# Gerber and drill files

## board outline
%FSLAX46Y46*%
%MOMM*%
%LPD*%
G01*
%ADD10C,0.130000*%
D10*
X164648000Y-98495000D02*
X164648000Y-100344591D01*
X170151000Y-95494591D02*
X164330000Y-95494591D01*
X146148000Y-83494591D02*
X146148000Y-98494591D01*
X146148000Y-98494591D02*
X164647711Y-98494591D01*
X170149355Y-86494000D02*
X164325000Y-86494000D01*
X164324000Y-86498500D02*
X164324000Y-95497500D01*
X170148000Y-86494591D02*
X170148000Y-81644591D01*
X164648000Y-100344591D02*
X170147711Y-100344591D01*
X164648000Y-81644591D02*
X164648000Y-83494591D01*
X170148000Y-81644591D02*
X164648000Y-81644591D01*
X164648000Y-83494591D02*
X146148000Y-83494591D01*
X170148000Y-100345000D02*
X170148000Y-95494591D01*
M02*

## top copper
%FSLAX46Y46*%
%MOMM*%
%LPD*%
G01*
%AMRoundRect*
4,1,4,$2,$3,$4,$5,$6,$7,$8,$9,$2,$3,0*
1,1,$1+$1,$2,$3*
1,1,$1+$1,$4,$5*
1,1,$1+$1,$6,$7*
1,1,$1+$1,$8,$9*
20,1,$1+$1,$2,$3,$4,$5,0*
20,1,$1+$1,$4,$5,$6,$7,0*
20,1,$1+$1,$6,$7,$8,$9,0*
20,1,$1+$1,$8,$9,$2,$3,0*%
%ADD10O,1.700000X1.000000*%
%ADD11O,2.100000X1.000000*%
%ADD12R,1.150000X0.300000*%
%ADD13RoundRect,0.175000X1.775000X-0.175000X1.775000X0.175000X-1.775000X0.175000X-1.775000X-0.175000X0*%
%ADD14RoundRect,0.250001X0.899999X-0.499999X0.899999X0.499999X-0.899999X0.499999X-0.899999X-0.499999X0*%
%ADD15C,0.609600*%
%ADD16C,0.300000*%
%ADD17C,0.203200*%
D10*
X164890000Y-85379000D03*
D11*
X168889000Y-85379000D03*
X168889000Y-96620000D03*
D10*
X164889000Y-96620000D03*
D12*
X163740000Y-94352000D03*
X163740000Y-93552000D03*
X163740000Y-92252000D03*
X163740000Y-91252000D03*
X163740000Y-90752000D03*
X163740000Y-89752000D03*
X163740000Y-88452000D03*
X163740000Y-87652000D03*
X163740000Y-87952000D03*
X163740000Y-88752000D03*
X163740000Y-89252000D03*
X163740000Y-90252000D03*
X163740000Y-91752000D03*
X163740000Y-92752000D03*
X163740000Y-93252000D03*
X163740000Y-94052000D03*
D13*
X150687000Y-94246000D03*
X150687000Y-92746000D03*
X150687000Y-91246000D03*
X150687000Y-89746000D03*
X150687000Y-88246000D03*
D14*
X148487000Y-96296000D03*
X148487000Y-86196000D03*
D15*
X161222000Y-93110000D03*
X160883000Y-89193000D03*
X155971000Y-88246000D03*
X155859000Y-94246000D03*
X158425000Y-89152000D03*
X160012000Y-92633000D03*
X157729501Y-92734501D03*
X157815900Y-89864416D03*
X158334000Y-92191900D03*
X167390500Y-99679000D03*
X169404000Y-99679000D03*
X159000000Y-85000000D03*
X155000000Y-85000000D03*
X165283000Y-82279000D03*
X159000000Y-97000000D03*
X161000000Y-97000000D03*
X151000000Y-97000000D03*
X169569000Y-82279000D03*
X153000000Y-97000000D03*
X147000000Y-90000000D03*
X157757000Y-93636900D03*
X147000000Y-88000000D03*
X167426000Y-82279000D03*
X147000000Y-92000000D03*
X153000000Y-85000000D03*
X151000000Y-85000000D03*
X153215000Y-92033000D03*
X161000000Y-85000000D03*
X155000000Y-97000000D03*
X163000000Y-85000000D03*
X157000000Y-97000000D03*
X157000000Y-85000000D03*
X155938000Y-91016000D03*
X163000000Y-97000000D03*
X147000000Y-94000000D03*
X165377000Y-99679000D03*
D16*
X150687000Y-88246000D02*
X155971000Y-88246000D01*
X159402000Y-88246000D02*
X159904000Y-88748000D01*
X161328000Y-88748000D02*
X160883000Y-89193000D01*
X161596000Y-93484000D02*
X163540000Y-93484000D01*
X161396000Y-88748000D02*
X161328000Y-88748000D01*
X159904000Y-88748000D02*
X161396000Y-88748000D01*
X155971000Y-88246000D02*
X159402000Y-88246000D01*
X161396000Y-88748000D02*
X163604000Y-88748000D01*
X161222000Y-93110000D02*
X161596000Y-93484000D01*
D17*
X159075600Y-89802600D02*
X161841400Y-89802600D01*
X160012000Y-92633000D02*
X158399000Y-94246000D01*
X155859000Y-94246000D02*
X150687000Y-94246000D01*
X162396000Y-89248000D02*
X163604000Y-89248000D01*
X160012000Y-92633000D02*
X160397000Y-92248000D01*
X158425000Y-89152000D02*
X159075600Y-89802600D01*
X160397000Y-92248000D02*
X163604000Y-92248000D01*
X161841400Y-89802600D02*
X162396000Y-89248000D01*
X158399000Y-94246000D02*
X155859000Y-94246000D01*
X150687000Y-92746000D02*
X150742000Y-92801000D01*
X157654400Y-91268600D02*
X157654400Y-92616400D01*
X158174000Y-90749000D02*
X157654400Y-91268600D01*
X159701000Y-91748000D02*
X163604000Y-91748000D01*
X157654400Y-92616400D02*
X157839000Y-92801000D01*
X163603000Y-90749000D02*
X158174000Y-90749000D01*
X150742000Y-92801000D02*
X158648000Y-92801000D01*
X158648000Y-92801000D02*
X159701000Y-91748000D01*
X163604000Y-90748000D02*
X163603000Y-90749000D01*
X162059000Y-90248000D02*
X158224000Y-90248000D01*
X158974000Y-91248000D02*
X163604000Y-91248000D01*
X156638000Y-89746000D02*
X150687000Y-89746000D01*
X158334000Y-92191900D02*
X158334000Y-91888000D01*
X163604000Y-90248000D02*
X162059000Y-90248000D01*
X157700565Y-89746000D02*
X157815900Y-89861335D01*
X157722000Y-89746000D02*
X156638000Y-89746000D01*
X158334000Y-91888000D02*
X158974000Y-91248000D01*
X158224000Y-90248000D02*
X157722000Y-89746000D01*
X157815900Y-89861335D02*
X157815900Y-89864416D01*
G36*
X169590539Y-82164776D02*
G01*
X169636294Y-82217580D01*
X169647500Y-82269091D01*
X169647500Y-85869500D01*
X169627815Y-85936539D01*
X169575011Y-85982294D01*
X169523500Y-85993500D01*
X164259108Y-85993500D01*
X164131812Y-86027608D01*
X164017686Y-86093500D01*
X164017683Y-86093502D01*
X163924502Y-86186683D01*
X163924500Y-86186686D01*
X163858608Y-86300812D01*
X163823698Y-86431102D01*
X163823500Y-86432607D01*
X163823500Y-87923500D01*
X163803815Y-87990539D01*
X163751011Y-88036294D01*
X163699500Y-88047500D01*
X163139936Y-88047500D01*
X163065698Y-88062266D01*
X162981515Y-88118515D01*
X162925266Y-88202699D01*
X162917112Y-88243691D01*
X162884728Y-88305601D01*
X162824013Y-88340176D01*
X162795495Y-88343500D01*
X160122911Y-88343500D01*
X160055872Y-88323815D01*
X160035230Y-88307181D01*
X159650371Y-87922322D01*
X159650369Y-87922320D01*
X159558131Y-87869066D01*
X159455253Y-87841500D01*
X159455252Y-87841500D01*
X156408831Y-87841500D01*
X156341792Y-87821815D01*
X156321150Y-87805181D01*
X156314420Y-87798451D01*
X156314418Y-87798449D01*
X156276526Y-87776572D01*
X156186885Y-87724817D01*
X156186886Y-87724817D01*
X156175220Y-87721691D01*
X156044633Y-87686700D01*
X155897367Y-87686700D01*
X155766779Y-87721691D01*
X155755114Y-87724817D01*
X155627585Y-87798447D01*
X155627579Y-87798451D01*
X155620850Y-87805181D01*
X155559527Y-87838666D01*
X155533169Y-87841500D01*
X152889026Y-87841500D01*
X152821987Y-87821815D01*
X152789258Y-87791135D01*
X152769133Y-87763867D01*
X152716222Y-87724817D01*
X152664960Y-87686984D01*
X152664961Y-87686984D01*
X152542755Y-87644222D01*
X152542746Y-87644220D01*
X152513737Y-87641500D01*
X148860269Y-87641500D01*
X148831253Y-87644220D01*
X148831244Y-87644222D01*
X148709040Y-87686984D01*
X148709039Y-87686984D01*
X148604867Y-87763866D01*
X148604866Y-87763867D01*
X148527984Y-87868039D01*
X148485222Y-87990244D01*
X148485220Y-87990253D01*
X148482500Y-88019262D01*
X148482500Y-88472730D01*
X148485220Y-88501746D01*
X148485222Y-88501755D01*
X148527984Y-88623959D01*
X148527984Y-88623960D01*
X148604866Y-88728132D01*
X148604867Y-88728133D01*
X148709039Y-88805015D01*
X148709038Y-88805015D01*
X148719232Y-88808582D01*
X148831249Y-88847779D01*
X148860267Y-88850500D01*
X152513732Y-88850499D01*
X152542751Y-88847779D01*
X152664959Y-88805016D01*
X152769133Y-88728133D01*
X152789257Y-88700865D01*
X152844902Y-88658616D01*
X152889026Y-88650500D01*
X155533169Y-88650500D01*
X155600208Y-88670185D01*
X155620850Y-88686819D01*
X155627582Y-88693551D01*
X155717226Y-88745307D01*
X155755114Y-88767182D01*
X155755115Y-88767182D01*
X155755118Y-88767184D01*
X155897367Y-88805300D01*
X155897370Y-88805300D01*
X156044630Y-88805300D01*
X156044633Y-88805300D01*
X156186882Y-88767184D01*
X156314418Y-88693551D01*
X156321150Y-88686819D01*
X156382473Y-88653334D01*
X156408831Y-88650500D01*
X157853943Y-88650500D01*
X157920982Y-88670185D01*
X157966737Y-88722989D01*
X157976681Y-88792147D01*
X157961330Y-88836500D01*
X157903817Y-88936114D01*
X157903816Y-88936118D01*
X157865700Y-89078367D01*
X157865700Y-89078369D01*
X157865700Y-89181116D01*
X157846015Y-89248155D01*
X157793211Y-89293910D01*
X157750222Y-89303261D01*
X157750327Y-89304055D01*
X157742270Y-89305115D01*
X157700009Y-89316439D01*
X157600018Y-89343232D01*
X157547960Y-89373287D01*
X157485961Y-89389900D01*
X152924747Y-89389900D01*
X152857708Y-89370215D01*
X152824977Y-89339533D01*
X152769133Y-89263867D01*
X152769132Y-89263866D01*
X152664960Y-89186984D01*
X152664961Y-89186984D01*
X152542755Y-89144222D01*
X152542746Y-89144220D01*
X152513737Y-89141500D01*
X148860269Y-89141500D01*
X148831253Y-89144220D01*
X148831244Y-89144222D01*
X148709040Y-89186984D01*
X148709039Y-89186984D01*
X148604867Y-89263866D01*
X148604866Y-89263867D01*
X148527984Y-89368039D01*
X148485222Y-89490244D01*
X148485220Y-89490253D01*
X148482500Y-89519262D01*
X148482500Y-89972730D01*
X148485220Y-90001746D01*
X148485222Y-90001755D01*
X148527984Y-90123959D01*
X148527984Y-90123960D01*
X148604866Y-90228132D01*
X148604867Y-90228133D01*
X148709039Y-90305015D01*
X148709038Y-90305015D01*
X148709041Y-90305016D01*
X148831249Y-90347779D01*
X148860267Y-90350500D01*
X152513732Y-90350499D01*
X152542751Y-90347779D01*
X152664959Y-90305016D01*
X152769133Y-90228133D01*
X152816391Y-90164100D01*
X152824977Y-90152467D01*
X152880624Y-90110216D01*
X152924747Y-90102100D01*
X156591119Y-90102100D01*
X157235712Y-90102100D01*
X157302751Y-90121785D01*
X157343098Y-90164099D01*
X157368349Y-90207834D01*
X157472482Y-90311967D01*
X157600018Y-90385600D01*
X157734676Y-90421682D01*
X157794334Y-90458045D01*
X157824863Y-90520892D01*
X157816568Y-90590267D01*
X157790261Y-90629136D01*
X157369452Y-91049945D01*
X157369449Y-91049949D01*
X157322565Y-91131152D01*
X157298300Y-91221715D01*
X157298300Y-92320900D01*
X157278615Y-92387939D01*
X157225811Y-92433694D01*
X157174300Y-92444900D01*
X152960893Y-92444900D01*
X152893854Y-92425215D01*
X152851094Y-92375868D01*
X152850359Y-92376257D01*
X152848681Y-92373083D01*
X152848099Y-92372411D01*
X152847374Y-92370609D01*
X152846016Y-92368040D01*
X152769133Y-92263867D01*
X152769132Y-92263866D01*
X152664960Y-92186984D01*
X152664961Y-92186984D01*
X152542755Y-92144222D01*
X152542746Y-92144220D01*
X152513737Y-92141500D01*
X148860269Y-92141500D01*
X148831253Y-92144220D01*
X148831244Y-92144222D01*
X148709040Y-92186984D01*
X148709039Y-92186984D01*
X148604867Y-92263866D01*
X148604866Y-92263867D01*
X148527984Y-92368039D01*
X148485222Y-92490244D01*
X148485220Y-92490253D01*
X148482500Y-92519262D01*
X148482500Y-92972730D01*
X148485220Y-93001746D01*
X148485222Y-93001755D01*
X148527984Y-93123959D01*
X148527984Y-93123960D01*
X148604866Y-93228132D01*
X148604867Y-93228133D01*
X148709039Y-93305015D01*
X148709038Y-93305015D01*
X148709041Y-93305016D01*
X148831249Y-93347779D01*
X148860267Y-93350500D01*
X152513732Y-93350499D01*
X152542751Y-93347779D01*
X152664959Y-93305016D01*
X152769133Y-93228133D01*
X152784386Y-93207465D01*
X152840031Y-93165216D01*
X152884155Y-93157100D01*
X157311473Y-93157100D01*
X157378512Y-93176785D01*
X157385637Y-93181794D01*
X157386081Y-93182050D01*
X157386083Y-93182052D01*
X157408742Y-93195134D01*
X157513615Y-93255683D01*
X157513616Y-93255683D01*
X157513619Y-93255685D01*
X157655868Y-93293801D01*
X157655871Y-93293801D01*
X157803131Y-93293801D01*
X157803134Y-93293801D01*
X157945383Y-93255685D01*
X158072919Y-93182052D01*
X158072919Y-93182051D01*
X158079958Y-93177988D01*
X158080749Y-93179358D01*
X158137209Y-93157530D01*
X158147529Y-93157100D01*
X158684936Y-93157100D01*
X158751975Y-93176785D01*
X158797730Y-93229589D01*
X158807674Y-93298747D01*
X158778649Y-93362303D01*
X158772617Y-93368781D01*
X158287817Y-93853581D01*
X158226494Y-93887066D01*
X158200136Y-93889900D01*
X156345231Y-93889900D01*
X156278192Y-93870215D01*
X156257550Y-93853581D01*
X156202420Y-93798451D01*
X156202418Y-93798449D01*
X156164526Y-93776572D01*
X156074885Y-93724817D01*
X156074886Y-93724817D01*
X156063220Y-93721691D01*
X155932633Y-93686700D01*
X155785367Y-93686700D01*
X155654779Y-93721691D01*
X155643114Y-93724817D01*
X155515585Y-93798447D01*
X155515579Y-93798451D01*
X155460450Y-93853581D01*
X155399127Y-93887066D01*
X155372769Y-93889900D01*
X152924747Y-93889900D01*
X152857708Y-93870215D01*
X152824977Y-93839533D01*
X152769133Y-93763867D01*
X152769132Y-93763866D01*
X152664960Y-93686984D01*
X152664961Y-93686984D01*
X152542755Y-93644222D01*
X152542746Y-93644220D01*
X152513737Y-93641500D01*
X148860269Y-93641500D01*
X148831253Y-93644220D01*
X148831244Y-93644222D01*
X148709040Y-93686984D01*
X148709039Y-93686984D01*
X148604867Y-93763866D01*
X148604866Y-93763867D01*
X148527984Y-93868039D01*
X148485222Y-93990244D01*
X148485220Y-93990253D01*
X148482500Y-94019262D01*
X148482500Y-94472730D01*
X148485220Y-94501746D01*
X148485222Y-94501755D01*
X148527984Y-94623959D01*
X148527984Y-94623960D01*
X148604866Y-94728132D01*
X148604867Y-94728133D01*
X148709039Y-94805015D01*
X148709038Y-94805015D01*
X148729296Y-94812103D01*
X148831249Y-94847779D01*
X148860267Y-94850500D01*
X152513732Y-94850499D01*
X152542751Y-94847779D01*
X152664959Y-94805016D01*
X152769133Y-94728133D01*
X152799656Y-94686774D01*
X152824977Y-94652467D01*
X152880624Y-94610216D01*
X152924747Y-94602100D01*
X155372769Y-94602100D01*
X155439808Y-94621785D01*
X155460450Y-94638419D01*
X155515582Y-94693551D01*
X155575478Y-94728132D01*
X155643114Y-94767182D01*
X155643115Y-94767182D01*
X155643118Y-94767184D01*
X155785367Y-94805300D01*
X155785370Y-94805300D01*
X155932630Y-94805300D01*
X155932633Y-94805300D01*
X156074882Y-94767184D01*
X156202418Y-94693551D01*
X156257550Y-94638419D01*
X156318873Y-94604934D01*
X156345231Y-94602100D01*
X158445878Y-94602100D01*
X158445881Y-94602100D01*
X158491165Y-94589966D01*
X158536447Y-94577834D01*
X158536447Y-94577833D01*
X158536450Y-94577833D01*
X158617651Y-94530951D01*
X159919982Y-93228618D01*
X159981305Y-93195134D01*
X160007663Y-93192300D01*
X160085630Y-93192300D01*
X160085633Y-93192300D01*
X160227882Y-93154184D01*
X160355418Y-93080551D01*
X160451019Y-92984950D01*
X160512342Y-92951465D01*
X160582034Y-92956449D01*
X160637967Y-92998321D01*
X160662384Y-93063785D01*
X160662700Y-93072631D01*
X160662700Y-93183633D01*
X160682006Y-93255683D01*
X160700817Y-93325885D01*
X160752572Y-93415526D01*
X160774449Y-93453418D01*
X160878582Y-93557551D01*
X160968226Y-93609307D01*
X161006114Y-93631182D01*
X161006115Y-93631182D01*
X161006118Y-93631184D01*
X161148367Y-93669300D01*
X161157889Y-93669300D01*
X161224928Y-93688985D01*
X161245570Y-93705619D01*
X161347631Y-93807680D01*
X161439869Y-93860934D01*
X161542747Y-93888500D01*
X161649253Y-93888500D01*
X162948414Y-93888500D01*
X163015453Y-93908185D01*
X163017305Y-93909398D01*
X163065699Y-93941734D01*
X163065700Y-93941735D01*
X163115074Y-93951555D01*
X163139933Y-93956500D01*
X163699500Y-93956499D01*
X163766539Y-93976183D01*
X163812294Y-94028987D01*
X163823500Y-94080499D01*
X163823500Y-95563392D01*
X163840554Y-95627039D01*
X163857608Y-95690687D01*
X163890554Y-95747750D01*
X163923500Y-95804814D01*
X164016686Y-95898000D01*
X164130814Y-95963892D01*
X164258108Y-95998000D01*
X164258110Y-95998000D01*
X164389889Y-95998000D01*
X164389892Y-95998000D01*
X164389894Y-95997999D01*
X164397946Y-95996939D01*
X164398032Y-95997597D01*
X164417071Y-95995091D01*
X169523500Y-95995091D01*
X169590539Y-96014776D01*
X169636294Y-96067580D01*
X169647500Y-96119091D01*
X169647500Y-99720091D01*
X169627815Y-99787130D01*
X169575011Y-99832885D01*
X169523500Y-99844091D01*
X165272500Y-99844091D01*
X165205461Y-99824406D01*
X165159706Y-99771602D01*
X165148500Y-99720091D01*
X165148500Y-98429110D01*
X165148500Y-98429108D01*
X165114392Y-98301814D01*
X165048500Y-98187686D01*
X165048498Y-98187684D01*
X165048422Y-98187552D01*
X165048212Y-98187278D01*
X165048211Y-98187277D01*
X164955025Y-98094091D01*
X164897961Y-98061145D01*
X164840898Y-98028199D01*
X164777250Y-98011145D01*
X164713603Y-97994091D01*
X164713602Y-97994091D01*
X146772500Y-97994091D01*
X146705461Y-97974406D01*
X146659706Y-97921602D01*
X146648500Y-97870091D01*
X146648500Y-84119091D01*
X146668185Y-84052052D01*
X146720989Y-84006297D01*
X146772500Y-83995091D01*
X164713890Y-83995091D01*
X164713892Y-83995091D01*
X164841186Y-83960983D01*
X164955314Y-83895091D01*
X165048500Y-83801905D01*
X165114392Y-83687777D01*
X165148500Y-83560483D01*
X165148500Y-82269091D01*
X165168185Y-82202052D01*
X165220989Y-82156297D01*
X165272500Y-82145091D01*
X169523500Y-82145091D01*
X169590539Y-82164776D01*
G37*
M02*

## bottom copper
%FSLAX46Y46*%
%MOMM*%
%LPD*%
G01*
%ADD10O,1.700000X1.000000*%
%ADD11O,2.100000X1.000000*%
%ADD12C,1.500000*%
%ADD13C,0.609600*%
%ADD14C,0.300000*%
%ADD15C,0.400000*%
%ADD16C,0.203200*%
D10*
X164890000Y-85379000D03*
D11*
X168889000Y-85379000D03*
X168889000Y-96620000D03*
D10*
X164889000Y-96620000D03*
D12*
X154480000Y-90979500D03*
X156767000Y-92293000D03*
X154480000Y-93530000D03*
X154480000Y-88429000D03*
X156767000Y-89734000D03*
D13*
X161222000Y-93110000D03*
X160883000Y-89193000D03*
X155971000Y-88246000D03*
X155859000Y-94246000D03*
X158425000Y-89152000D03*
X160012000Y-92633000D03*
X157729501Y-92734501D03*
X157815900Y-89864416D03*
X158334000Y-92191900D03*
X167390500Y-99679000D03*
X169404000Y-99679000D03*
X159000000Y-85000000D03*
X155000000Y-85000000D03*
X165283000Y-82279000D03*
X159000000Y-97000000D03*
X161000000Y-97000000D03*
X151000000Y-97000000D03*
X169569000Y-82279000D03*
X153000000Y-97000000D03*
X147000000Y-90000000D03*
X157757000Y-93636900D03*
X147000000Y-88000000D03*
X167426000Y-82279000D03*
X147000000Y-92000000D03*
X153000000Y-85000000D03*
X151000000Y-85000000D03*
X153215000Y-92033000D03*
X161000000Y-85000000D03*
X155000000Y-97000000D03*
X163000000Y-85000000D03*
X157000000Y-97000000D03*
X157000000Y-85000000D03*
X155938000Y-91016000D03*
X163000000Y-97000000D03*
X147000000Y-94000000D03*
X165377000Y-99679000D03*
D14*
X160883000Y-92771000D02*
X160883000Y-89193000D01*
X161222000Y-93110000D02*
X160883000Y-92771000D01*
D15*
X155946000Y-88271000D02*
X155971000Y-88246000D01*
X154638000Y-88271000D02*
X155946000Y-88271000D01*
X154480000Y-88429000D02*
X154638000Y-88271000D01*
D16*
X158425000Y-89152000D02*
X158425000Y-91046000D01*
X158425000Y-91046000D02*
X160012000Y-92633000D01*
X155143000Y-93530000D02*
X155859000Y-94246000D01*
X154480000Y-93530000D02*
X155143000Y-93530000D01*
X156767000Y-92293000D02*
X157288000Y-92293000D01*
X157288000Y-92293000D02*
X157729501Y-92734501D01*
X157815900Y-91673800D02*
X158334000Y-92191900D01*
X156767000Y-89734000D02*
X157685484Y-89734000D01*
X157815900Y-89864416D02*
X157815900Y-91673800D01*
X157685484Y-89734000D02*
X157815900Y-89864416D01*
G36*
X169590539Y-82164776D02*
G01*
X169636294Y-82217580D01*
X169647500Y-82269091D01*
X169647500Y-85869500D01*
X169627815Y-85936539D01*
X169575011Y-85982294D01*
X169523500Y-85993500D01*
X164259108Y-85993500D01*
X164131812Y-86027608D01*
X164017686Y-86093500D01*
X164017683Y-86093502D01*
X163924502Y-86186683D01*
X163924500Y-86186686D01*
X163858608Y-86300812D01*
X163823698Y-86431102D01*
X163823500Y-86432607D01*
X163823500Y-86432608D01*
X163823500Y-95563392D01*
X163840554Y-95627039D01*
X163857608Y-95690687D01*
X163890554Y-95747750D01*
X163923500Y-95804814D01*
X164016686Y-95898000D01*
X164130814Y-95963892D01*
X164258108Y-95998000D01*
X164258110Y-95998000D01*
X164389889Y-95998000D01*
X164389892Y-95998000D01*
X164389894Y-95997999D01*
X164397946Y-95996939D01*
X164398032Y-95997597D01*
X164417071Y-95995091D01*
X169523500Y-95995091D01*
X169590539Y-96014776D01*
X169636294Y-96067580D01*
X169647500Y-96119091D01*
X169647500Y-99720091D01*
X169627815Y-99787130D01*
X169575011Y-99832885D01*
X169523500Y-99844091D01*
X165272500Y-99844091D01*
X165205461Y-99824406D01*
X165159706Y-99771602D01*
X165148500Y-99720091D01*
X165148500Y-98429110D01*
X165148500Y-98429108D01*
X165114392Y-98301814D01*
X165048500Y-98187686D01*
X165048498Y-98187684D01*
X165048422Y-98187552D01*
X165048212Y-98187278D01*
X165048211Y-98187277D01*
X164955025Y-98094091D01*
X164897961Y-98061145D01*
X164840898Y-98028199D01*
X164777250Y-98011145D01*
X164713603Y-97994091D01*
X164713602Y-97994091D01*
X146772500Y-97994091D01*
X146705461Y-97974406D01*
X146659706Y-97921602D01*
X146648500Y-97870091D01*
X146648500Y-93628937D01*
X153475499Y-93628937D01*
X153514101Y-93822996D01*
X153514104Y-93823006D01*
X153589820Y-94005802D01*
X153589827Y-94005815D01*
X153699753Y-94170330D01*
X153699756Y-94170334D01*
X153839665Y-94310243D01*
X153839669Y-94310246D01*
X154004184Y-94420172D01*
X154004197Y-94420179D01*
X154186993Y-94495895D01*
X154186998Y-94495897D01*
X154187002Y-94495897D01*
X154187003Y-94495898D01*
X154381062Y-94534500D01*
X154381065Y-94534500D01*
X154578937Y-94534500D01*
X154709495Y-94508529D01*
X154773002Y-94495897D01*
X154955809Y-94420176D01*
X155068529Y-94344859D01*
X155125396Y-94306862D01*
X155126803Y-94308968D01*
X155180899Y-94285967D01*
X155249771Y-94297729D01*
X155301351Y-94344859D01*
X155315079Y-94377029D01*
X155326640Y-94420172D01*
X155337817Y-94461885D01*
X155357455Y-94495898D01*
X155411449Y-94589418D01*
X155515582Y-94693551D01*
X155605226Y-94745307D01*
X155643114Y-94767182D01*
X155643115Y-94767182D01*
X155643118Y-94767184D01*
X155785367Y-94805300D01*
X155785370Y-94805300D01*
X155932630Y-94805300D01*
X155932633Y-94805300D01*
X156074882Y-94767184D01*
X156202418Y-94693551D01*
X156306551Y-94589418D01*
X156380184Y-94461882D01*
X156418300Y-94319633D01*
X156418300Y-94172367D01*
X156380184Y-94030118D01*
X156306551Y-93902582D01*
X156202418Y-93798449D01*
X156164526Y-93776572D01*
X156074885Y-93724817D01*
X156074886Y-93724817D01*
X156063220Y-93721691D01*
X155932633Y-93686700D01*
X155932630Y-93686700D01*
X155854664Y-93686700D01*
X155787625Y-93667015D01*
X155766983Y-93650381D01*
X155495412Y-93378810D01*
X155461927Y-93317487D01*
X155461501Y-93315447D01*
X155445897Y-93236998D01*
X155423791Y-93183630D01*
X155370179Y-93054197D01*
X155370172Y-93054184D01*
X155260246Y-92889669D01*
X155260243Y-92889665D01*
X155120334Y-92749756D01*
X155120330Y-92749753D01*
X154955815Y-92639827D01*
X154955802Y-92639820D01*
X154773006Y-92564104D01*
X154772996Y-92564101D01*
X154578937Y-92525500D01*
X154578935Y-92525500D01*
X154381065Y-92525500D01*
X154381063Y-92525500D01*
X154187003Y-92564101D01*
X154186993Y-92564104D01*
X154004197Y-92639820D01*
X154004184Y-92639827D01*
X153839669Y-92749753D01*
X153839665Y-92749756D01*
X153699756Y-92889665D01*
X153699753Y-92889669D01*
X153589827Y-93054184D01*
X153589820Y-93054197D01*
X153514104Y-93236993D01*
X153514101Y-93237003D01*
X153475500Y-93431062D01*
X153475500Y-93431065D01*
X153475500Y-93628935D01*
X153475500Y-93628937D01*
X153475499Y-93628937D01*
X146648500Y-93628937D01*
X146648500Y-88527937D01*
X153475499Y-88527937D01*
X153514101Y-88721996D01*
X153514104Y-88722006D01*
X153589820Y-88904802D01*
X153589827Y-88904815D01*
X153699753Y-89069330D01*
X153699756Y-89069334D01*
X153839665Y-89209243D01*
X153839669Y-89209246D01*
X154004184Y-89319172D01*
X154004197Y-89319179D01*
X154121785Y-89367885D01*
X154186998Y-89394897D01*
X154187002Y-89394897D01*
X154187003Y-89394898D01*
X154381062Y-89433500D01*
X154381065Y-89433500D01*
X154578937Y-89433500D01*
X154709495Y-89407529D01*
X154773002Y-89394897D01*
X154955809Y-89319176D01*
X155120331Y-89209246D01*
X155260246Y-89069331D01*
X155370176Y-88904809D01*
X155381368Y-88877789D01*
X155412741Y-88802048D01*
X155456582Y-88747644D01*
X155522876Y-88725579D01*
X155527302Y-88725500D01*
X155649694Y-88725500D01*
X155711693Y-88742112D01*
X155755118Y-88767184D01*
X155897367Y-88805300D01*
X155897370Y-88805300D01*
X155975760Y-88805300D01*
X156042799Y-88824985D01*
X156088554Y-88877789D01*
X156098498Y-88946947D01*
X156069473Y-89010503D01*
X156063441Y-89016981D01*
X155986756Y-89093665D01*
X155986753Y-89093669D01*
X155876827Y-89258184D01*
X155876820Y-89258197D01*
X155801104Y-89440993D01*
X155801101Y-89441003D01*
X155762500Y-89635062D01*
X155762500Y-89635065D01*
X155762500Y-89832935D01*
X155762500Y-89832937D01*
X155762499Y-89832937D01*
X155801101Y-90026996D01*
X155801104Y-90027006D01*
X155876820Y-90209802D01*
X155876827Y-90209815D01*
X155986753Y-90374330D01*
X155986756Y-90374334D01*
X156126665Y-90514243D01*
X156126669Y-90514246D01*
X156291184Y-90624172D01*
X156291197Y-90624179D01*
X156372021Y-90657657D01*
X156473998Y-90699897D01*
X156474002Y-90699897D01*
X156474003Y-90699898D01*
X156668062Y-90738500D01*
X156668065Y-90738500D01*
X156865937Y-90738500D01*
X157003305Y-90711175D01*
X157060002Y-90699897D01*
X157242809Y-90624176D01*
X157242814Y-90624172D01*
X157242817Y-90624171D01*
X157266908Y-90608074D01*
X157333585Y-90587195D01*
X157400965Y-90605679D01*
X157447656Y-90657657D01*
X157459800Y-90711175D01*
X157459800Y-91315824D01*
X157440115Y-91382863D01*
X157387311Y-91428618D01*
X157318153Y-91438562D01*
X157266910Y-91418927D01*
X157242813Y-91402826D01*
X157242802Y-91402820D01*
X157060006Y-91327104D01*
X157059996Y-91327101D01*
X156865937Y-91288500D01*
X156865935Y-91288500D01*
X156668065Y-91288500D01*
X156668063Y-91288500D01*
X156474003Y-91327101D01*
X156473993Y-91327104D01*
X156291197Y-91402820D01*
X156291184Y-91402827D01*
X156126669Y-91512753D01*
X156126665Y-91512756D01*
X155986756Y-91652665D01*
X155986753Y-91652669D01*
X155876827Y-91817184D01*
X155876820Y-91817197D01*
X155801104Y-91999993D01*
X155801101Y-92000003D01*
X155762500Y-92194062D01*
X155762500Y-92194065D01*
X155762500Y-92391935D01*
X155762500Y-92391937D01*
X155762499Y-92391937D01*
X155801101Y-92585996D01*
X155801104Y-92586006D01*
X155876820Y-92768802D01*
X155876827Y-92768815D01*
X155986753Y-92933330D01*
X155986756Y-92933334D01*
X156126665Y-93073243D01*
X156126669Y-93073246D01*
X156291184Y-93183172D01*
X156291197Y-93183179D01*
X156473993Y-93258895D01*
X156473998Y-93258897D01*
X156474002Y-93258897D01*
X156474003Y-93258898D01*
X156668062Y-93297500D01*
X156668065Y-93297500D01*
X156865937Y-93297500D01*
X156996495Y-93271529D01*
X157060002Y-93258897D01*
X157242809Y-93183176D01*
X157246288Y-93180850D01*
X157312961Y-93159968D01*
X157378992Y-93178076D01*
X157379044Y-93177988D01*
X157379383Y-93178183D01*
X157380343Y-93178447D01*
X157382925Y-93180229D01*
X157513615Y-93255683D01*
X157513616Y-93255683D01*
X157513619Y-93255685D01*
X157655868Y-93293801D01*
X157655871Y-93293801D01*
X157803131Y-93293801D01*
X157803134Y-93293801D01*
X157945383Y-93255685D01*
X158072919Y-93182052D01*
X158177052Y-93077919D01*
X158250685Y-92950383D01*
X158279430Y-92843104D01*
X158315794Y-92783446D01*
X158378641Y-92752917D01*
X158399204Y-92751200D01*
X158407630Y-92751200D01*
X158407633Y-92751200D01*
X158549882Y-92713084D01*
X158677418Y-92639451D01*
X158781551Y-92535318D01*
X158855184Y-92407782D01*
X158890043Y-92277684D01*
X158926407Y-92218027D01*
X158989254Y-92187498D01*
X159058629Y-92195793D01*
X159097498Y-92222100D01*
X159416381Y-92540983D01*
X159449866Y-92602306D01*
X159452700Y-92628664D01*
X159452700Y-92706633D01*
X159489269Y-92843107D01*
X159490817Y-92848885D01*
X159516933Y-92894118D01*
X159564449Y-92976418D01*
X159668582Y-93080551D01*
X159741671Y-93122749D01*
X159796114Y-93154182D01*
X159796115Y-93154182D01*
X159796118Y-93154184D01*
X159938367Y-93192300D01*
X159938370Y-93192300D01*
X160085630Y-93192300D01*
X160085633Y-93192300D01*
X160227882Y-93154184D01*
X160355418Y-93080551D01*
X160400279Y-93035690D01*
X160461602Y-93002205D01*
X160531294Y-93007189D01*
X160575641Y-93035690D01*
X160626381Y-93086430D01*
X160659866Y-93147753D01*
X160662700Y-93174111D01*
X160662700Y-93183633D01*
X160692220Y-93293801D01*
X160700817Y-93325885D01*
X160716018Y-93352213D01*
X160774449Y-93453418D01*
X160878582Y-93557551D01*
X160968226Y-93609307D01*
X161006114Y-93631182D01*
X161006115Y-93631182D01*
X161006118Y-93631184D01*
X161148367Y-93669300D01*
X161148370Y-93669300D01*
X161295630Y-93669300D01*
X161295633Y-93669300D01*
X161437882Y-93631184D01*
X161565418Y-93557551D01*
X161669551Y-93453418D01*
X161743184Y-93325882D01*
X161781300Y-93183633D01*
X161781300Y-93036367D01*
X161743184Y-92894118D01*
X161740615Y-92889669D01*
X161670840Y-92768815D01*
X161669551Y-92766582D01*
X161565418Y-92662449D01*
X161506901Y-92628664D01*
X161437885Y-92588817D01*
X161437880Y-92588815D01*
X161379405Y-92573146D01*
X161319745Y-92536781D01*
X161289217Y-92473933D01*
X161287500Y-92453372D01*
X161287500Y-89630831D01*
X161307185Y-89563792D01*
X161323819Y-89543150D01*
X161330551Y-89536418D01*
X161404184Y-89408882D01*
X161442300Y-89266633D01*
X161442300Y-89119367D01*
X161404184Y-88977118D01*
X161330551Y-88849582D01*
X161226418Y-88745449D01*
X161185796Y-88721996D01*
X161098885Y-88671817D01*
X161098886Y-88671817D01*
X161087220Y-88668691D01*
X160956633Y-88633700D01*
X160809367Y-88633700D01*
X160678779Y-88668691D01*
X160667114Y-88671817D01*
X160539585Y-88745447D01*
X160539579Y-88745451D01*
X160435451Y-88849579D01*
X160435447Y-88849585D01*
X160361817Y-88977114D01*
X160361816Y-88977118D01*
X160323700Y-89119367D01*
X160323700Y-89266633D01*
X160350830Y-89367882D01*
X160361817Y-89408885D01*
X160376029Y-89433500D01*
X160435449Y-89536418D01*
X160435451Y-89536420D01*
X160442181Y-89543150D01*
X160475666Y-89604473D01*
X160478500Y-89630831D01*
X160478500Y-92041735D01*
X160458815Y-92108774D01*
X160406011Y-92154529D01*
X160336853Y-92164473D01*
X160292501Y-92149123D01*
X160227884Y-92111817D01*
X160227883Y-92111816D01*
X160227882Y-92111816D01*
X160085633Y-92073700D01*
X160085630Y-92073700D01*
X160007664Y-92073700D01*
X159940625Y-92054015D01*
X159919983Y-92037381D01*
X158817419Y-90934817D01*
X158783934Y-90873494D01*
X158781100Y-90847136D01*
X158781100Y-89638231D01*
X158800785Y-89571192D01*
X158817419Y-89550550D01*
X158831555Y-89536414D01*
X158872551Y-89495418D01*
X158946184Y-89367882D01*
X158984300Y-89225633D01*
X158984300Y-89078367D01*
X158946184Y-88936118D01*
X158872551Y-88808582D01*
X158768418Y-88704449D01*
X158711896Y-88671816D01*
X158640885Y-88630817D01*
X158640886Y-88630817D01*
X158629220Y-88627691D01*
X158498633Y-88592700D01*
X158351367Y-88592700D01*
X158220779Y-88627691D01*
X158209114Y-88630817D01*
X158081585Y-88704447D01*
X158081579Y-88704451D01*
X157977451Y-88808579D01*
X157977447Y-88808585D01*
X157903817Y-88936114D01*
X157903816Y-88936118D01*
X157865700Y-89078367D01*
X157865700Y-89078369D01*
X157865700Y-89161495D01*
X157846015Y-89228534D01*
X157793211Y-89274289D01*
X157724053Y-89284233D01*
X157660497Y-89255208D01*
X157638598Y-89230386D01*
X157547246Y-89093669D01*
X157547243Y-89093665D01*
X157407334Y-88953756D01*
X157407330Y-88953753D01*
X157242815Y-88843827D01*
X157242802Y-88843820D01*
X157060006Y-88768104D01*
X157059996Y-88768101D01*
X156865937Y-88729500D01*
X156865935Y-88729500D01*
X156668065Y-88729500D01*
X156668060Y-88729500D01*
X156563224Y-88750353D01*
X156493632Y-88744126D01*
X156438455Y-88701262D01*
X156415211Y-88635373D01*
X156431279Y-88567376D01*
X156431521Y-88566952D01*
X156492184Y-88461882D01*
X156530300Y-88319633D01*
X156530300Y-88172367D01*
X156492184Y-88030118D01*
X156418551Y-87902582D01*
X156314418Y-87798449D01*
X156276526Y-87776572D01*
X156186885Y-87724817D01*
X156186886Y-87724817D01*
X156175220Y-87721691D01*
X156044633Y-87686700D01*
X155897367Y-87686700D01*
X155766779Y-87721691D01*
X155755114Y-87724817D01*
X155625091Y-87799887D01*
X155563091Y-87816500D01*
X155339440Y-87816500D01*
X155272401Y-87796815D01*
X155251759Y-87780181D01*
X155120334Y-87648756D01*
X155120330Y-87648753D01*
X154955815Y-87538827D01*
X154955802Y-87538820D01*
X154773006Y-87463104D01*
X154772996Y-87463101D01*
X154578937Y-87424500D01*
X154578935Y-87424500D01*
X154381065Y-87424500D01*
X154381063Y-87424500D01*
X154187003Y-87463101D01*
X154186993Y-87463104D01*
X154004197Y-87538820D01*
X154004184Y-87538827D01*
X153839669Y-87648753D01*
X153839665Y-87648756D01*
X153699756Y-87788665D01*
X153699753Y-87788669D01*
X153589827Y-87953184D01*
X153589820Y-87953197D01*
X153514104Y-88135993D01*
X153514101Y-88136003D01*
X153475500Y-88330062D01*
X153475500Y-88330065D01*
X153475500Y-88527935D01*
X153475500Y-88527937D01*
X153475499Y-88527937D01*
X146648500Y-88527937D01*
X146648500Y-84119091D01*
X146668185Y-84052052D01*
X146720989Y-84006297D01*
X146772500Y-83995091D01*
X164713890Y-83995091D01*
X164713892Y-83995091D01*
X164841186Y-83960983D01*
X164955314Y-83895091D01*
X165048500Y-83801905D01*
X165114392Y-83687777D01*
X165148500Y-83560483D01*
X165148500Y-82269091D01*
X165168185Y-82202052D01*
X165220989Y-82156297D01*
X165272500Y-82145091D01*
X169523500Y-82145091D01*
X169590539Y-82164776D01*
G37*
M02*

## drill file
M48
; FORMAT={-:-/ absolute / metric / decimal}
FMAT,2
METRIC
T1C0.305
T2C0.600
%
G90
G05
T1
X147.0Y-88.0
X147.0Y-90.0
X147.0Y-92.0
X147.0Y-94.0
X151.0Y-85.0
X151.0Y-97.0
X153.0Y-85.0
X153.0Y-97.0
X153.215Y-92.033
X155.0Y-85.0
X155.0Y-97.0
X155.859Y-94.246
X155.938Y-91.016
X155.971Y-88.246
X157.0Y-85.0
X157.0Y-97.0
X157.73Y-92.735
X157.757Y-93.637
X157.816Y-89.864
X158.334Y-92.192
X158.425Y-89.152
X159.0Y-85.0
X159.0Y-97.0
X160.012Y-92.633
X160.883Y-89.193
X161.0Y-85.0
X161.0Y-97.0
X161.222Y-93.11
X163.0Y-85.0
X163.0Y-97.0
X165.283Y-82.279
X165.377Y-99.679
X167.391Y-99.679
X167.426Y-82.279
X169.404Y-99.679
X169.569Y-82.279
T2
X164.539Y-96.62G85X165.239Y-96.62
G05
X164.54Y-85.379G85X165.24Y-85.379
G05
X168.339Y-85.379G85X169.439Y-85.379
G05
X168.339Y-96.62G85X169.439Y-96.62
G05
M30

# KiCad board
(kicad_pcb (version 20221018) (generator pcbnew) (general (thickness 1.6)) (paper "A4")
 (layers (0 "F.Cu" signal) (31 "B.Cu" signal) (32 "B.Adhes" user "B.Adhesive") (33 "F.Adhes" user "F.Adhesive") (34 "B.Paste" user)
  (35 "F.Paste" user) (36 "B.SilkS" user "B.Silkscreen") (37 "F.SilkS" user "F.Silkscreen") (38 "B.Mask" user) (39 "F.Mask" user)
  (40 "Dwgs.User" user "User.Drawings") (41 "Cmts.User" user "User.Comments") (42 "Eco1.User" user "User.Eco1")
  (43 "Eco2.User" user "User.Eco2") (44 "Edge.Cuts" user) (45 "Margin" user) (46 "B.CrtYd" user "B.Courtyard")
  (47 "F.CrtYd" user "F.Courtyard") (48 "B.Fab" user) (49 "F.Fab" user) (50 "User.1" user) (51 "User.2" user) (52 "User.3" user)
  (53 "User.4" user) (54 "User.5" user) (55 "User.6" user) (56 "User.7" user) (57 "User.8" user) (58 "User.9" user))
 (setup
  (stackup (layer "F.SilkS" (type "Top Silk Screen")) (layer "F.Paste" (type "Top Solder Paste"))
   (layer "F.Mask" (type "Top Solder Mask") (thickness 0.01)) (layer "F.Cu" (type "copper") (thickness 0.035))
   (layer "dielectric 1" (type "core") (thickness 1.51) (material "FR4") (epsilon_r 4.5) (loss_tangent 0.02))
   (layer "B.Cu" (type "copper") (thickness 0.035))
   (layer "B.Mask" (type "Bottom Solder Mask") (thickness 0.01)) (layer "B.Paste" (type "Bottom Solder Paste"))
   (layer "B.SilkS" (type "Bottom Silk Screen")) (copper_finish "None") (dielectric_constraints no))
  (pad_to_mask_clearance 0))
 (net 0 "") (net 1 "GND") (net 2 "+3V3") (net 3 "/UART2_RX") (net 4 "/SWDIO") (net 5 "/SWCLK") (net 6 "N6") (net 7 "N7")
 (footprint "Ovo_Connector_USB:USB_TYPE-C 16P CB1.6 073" (layer "F.Cu") (at 167.41 91.002 90)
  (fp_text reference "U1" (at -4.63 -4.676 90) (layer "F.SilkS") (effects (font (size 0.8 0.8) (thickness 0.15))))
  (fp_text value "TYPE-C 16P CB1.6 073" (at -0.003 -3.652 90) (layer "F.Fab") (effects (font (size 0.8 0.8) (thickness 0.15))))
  (pad "25" thru_hole oval (at 5.623 -2.52 90) (size 1 1.7) (drill oval 0.6 1.3) (layers "*.Cu" "*.Mask") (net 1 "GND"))
  (pad "26" thru_hole oval (at 5.623 1.479 90) (size 1 2.1) (drill oval 0.6 1.7) (layers "*.Cu" "*.Mask") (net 1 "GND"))
  (pad "27" thru_hole oval (at -5.618 1.479 90) (size 1 2.1) (drill oval 0.6 1.7) (layers "*.Cu" "*.Mask") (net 1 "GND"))
  (pad "28" thru_hole oval (at -5.618 -2.521 90) (size 1 1.7) (drill oval 0.6 1.3) (layers "*.Cu" "*.Mask") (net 1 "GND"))
  (pad "A1" smd rect (at -3.35 -3.67 90) (size 0.3 1.15) (layers "F.Cu" "F.Paste" "F.Mask") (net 1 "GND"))
  (pad "A4" smd rect (at -2.55 -3.67 90) (size 0.3 1.15) (layers "F.Cu" "F.Paste" "F.Mask") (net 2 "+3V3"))
  (pad "A5" smd rect (at -1.25 -3.67 90) (size 0.3 1.15) (layers "F.Cu" "F.Paste" "F.Mask") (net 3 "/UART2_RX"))
  (pad "A6" smd rect (at -0.25 -3.67 90) (size 0.3 1.15) (layers "F.Cu" "F.Paste" "F.Mask") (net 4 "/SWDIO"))
  (pad "A7" smd rect (at 0.25 -3.67 90) (size 0.3 1.15) (layers "F.Cu" "F.Paste" "F.Mask") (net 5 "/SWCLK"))
  (pad "A8" smd rect (at 1.25 -3.67 90) (size 0.3 1.15) (layers "F.Cu" "F.Paste" "F.Mask") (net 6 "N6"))
  (pad "A9" smd rect (at 2.55 -3.67 90) (size 0.3 1.15) (layers "F.Cu" "F.Paste" "F.Mask") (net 2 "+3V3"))
  (pad "A12" smd rect (at 3.35 -3.67 90) (size 0.3 1.15) (layers "F.Cu" "F.Paste" "F.Mask") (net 1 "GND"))
  (pad "B1" smd rect (at 3.05 -3.67 90) (size 0.3 1.15) (layers "F.Cu" "F.Paste" "F.Mask") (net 1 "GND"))
  (pad "B4" smd rect (at 2.25 -3.67 90) (size 0.3 1.15) (layers "F.Cu" "F.Paste" "F.Mask") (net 2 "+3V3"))
  (pad "B5" smd rect (at 1.75 -3.67 90) (size 0.3 1.15) (layers "F.Cu" "F.Paste" "F.Mask") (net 3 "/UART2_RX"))
  (pad "B6" smd rect (at 0.75 -3.67 90) (size 0.3 1.15) (layers "F.Cu" "F.Paste" "F.Mask") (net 4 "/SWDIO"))
  (pad "B7" smd rect (at -0.75 -3.67 90) (size 0.3 1.15) (layers "F.Cu" "F.Paste" "F.Mask") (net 5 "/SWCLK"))
  (pad "B8" smd rect (at -1.75 -3.67 90) (size 0.3 1.15) (layers "F.Cu" "F.Paste" "F.Mask") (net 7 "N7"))
  (pad "B9" smd rect (at -2.25 -3.67 90) (size 0.3 1.15) (layers "F.Cu" "F.Paste" "F.Mask") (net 2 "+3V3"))
  (pad "B12" smd rect (at -3.05 -3.67 90) (size 0.3 1.15) (layers "F.Cu" "F.Paste" "F.Mask") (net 1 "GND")))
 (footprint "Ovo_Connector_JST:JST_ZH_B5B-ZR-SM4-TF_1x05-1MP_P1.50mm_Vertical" (layer "F.Cu") (at 149.987 91.246 90)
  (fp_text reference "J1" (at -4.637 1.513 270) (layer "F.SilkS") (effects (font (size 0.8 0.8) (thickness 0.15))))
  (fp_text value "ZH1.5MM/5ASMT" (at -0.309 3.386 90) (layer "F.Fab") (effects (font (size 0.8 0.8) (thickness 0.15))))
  (pad "1" smd roundrect (at -3 0.7 90) (size 0.7 3.9) (layers "F.Cu" "F.Paste" "F.Mask") (roundrect_rratio 0.25) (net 3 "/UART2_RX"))
  (pad "2" smd roundrect (at -1.5 0.7 90) (size 0.7 3.9) (layers "F.Cu" "F.Paste" "F.Mask") (roundrect_rratio 0.25) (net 5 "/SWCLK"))
  (pad "3" smd roundrect (at 0 0.7 90) (size 0.7 3.9) (layers "F.Cu" "F.Paste" "F.Mask") (roundrect_rratio 0.25) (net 1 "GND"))
  (pad "4" smd roundrect (at 1.5 0.7 90) (size 0.7 3.9) (layers "F.Cu" "F.Paste" "F.Mask") (roundrect_rratio 0.25) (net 4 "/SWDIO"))
  (pad "5" smd roundrect (at 3 0.7 90) (size 0.7 3.9) (layers "F.Cu" "F.Paste" "F.Mask") (roundrect_rratio 0.25) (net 2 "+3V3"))
  (pad "MP" smd roundrect (at -5.05 -1.5 90) (size 1.5 2.3) (layers "F.Cu" "F.Paste" "F.Mask") (roundrect_rratio 0.1666673333) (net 1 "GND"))
  (pad "MP" smd roundrect (at 5.05 -1.5 90) (size 1.5 2.3) (layers "F.Cu" "F.Paste" "F.Mask") (roundrect_rratio 0.1666673333) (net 1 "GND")))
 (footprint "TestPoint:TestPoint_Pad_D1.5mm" (layer "B.Cu") (at 154.48 90.9795 180)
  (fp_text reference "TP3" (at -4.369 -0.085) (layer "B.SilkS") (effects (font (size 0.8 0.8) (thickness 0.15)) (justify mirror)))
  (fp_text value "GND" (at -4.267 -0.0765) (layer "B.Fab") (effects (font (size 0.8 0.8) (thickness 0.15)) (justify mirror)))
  (pad "1" smd circle (at 0 0 180) (size 1.5 1.5) (layers "B.Cu" "B.Mask") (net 1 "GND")))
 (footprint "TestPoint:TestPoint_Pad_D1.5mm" (layer "B.Cu") (at 156.767 92.293 180)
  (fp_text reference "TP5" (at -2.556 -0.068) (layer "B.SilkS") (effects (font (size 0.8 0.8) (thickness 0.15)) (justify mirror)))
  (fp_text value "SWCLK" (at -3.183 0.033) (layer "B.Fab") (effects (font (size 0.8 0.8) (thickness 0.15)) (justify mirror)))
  (pad "1" smd circle (at 0 0 180) (size 1.5 1.5) (layers "B.Cu" "B.Mask") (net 5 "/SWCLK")))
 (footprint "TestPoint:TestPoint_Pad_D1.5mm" (layer "B.Cu") (at 154.48 93.53 180)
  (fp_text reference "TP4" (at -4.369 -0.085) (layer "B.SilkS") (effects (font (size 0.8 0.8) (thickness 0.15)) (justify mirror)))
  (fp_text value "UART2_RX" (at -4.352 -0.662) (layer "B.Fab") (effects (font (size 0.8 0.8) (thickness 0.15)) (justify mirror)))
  (pad "1" smd circle (at 0 0 180) (size 1.5 1.5) (layers "B.Cu" "B.Mask") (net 3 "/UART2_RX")))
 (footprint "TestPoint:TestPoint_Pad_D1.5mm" (layer "B.Cu") (at 154.48 88.429 180)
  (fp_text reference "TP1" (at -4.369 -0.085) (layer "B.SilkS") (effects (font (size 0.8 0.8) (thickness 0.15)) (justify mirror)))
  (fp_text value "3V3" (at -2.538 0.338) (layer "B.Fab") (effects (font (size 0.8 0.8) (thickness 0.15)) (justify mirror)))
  (pad "1" smd circle (at 0 0 180) (size 1.5 1.5) (layers "B.Cu" "B.Mask") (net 2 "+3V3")))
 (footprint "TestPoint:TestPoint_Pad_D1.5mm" (layer "B.Cu") (at 156.767 89.734 180)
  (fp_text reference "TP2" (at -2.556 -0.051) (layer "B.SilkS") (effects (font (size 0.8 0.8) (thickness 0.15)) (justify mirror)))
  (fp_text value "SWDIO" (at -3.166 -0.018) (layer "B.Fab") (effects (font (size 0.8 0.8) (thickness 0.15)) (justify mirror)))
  (pad "1" smd circle (at 0 0 180) (size 1.5 1.5) (layers "B.Cu" "B.Mask") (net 4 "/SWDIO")))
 (gr_line (start 164.648 98.495) (end 164.648 100.344591) (stroke (width 0.13) (type solid)) (layer "Edge.Cuts"))
 (gr_line (start 170.151 95.494591) (end 164.33 95.494591) (stroke (width 0.13) (type solid)) (layer "Edge.Cuts"))
 (gr_line (start 146.148 83.494591) (end 146.148 98.494591) (stroke (width 0.13) (type solid)) (layer "Edge.Cuts"))
 (gr_line (start 146.148 98.494591) (end 164.647711 98.494591) (stroke (width 0.13) (type solid)) (layer "Edge.Cuts"))
 (gr_line (start 170.149355 86.494) (end 164.325 86.494) (stroke (width 0.13) (type solid)) (layer "Edge.Cuts"))
 (gr_line (start 164.324 86.4985) (end 164.324 95.4975) (stroke (width 0.13) (type solid)) (layer "Edge.Cuts"))
 (gr_line (start 170.148 86.494591) (end 170.148 81.644591) (stroke (width 0.13) (type solid)) (layer "Edge.Cuts"))
 (gr_line (start 164.648 100.344591) (end 170.147711 100.344591) (stroke (width 0.13) (type solid)) (layer "Edge.Cuts"))
 (gr_line (start 164.648 81.644591) (end 164.648 83.494591) (stroke (width 0.13) (type solid)) (layer "Edge.Cuts"))
 (gr_line (start 170.148 81.644591) (end 164.648 81.644591) (stroke (width 0.13) (type solid)) (layer "Edge.Cuts"))
 (gr_line (start 164.648 83.494591) (end 146.148 83.494591) (stroke (width 0.13) (type solid)) (layer "Edge.Cuts"))
 (gr_line (start 170.148 100.345) (end 170.148 95.494591) (stroke (width 0.13) (type solid)) (layer "Edge.Cuts"))
 (segment (start 150.687 88.246) (end 155.971 88.246) (width 0.3) (layer "F.Cu") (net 2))
 (segment (start 159.402 88.246) (end 159.904 88.748) (width 0.3) (layer "F.Cu") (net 2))
 (segment (start 161.328 88.748) (end 160.883 89.193) (width 0.3) (layer "F.Cu") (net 2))
 (segment (start 161.596 93.484) (end 163.54 93.484) (width 0.3) (layer "F.Cu") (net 2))
 (segment (start 161.396 88.748) (end 161.328 88.748) (width 0.3) (layer "F.Cu") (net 2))
 (segment (start 159.904 88.748) (end 161.396 88.748) (width 0.3) (layer "F.Cu") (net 2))
 (segment (start 155.971 88.246) (end 159.402 88.246) (width 0.3) (layer "F.Cu") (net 2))
 (segment (start 161.396 88.748) (end 163.604 88.748) (width 0.3) (layer "F.Cu") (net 2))
 (segment (start 161.222 93.11) (end 161.596 93.484) (width 0.3) (layer "F.Cu") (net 2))
 (via (at 161.222 93.11) (size 0.6096) (drill 0.3048) (layers "F.Cu" "B.Cu") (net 2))
 (via (at 160.883 89.193) (size 0.6096) (drill 0.3048) (layers "F.Cu" "B.Cu") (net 2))
 (via (at 155.971 88.246) (size 0.6096) (drill 0.3048) (layers "F.Cu" "B.Cu") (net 2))
 (segment (start 160.883 92.771) (end 160.883 89.193) (width 0.3) (layer "B.Cu") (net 2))
 (segment (start 161.222 93.11) (end 160.883 92.771) (width 0.3) (layer "B.Cu") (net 2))
 (segment (start 155.946 88.271) (end 155.971 88.246) (width 0.4) (layer "B.Cu") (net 2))
 (segment (start 154.638 88.271) (end 155.946 88.271) (width 0.4) (layer "B.Cu") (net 2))
 (segment (start 154.48 88.429) (end 154.638 88.271) (width 0.4) (layer "B.Cu") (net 2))
 (segment (start 159.0756 89.8026) (end 161.8414 89.8026) (width 0.2032) (layer "F.Cu") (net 3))
 (segment (start 160.012 92.633) (end 158.399 94.246) (width 0.2032) (layer "F.Cu") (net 3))
 (segment (start 155.859 94.246) (end 150.687 94.246) (width 0.2032) (layer "F.Cu") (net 3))
 (segment (start 162.396 89.248) (end 163.604 89.248) (width 0.2032) (layer "F.Cu") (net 3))
 (segment (start 160.012 92.633) (end 160.397 92.248) (width 0.2032) (layer "F.Cu") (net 3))
 (segment (start 158.425 89.152) (end 159.0756 89.8026) (width 0.2032) (layer "F.Cu") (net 3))
 (segment (start 160.397 92.248) (end 163.604 92.248) (width 0.2032) (layer "F.Cu") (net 3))
 (segment (start 161.8414 89.8026) (end 162.396 89.248) (width 0.2032) (layer "F.Cu") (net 3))
 (segment (start 158.399 94.246) (end 155.859 94.246) (width 0.2032) (layer "F.Cu") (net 3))
 (via (at 155.859 94.246) (size 0.6096) (drill 0.3048) (layers "F.Cu" "B.Cu") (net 3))
 (via (at 158.425 89.152) (size 0.6096) (drill 0.3048) (layers "F.Cu" "B.Cu") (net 3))
 (via (at 160.012 92.633) (size 0.6096) (drill 0.3048) (layers "F.Cu" "B.Cu") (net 3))
 (segment (start 158.425 89.152) (end 158.425 91.046) (width 0.2032) (layer "B.Cu") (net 3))
 (segment (start 158.425 91.046) (end 160.012 92.633) (width 0.2032) (layer "B.Cu") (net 3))
 (segment (start 155.143 93.53) (end 155.859 94.246) (width 0.2032) (layer "B.Cu") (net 3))
 (segment (start 154.48 93.53) (end 155.143 93.53) (width 0.2032) (layer "B.Cu") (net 3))
 (segment (start 150.687 92.746) (end 150.742 92.801) (width 0.2032) (layer "F.Cu") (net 5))
 (segment (start 157.6544 91.2686) (end 157.6544 92.6164) (width 0.2032) (layer "F.Cu") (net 5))
 (segment (start 158.174 90.749) (end 157.6544 91.2686) (width 0.2032) (layer "F.Cu") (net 5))
 (segment (start 159.701 91.748) (end 163.604 91.748) (width 0.2032) (layer "F.Cu") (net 5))
 (segment (start 157.6544 92.6164) (end 157.839 92.801) (width 0.2032) (layer "F.Cu") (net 5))
 (segment (start 163.603 90.749) (end 158.174 90.749) (width 0.2032) (layer "F.Cu") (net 5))
 (segment (start 150.742 92.801) (end 158.648 92.801) (width 0.2032) (layer "F.Cu") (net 5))
 (segment (start 158.648 92.801) (end 159.701 91.748) (width 0.2032) (layer "F.Cu") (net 5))
 (segment (start 163.604 90.748) (end 163.603 90.749) (width 0.2032) (layer "F.Cu") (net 5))
 (via (at 157.729501 92.734501) (size 0.6096) (drill 0.3048) (layers "F.Cu" "B.Cu") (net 5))
 (segment (start 156.767 92.293) (end 157.288 92.293) (width 0.2032) (layer "B.Cu") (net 5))
 (segment (start 157.288 92.293) (end 157.729501 92.734501) (width 0.2032) (layer "B.Cu") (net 5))
 (segment (start 162.059 90.248) (end 158.224 90.248) (width 0.2032) (layer "F.Cu") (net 4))
 (segment (start 158.974 91.248) (end 163.604 91.248) (width 0.2032) (layer "F.Cu") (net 4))
 (segment (start 156.638 89.746) (end 150.687 89.746) (width 0.2032) (layer "F.Cu") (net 4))
 (segment (start 158.334 92.1919) (end 158.334 91.888) (width 0.2032) (layer "F.Cu") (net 4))
 (segment (start 163.604 90.248) (end 162.059 90.248) (width 0.2032) (layer "F.Cu") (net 4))
 (segment (start 157.700565 89.746) (end 157.8159 89.861335) (width 0.2032) (layer "F.Cu") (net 4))
 (segment (start 157.722 89.746) (end 156.638 89.746) (width 0.2032) (layer "F.Cu") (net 4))
 (segment (start 158.334 91.888) (end 158.974 91.248) (width 0.2032) (layer "F.Cu") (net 4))
 (segment (start 158.224 90.248) (end 157.722 89.746) (width 0.2032) (layer "F.Cu") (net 4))
 (segment (start 157.8159 89.861335) (end 157.8159 89.864416) (width 0.2032) (layer "F.Cu") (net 4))
 (via (at 157.8159 89.864416) (size 0.6096) (drill 0.3048) (layers "F.Cu" "B.Cu") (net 4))
 (via (at 158.334 92.1919) (size 0.6096) (drill 0.3048) (layers "F.Cu" "B.Cu") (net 4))
 (segment (start 157.8159 91.6738) (end 158.334 92.1919) (width 0.2032) (layer "B.Cu") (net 4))
 (segment (start 156.767 89.734) (end 157.685484 89.734) (width 0.2032) (layer "B.Cu") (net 4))
 (segment (start 157.8159 89.864416) (end 157.8159 91.6738) (width 0.2032) (layer "B.Cu") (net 4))
 (segment (start 157.685484 89.734) (end 157.8159 89.864416) (width 0.2032) (layer "B.Cu") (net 4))
 (via (at 167.3905 99.679) (size 0.6096) (drill 0.3048) (layers "F.Cu" "B.Cu") (free) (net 1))
 (via (at 169.404 99.679) (size 0.6096) (drill 0.3048) (layers "F.Cu" "B.Cu") (free) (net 1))
 (via (at 159 85) (size 0.6096) (drill 0.3048) (layers "F.Cu" "B.Cu") (free) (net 1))
 (via (at 155 85) (size 0.6096) (drill 0.3048) (layers "F.Cu" "B.Cu") (free) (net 1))
 (via (at 165.283 82.279) (size 0.6096) (drill 0.3048) (layers "F.Cu" "B.Cu") (free) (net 1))
 (via (at 159 97) (size 0.6096) (drill 0.3048) (layers "F.Cu" "B.Cu") (free) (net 1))
 (via (at 161 97) (size 0.6096) (drill 0.3048) (layers "F.Cu" "B.Cu") (free) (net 1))
 (via (at 151 97) (size 0.6096) (drill 0.3048) (layers "F.Cu" "B.Cu") (free) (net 1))
 (via (at 169.569 82.279) (size 0.6096) (drill 0.3048) (layers "F.Cu" "B.Cu") (free) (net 1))
 (via (at 153 97) (size 0.6096) (drill 0.3048) (layers "F.Cu" "B.Cu") (free) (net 1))
 (via (at 147 90) (size 0.6096) (drill 0.3048) (layers "F.Cu" "B.Cu") (free) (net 1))
 (via (at 157.757 93.6369) (size 0.6096) (drill 0.3048) (layers "F.Cu" "B.Cu") (free) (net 1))
 (via (at 147 88) (size 0.6096) (drill 0.3048) (layers "F.Cu" "B.Cu") (free) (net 1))
 (via (at 167.426 82.279) (size 0.6096) (drill 0.3048) (layers "F.Cu" "B.Cu") (free) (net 1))
 (via (at 147 92) (size 0.6096) (drill 0.3048) (layers "F.Cu" "B.Cu") (free) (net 1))
 (via (at 153 85) (size 0.6096) (drill 0.3048) (layers "F.Cu" "B.Cu") (free) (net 1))
 (via (at 151 85) (size 0.6096) (drill 0.3048) (layers "F.Cu" "B.Cu") (free) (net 1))
 (via (at 153.215 92.033) (size 0.6096) (drill 0.3048) (layers "F.Cu" "B.Cu") (free) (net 1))
 (via (at 161 85) (size 0.6096) (drill 0.3048) (layers "F.Cu" "B.Cu") (free) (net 1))
 (via (at 155 97) (size 0.6096) (drill 0.3048) (layers "F.Cu" "B.Cu") (free) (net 1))
 (via (at 163 85) (size 0.6096) (drill 0.3048) (layers "F.Cu" "B.Cu") (free) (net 1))
 (via (at 157 97) (size 0.6096) (drill 0.3048) (layers "F.Cu" "B.Cu") (free) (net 1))
 (via (at 157 85) (size 0.6096) (drill 0.3048) (layers "F.Cu" "B.Cu") (free) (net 1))
 (via (at 155.938 91.016) (size 0.6096) (drill 0.3048) (layers "F.Cu" "B.Cu") (free) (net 1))
 (via (at 163 97) (size 0.6096) (drill 0.3048) (layers "F.Cu" "B.Cu") (free) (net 1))
 (via (at 147 94) (size 0.6096) (drill 0.3048) (layers "F.Cu" "B.Cu") (free) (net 1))
 (via (at 165.377 99.679) (size 0.6096) (drill 0.3048) (layers "F.Cu" "B.Cu") (free) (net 1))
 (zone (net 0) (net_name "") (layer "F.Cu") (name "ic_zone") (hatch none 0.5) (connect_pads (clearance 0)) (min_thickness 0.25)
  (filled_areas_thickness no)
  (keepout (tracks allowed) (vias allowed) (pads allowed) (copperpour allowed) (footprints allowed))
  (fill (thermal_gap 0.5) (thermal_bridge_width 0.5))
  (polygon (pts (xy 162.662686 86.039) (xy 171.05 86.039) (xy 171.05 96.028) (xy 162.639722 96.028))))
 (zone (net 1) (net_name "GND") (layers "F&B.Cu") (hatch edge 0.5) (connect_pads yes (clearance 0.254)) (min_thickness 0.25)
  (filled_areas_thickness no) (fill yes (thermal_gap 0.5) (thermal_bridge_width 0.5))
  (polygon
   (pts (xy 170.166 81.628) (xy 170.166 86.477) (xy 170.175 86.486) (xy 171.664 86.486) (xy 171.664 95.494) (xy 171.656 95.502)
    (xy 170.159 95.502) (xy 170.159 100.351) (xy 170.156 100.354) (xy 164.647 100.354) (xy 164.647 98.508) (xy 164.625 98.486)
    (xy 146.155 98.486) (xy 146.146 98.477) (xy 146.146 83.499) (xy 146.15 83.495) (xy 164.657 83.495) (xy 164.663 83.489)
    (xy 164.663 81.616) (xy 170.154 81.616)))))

